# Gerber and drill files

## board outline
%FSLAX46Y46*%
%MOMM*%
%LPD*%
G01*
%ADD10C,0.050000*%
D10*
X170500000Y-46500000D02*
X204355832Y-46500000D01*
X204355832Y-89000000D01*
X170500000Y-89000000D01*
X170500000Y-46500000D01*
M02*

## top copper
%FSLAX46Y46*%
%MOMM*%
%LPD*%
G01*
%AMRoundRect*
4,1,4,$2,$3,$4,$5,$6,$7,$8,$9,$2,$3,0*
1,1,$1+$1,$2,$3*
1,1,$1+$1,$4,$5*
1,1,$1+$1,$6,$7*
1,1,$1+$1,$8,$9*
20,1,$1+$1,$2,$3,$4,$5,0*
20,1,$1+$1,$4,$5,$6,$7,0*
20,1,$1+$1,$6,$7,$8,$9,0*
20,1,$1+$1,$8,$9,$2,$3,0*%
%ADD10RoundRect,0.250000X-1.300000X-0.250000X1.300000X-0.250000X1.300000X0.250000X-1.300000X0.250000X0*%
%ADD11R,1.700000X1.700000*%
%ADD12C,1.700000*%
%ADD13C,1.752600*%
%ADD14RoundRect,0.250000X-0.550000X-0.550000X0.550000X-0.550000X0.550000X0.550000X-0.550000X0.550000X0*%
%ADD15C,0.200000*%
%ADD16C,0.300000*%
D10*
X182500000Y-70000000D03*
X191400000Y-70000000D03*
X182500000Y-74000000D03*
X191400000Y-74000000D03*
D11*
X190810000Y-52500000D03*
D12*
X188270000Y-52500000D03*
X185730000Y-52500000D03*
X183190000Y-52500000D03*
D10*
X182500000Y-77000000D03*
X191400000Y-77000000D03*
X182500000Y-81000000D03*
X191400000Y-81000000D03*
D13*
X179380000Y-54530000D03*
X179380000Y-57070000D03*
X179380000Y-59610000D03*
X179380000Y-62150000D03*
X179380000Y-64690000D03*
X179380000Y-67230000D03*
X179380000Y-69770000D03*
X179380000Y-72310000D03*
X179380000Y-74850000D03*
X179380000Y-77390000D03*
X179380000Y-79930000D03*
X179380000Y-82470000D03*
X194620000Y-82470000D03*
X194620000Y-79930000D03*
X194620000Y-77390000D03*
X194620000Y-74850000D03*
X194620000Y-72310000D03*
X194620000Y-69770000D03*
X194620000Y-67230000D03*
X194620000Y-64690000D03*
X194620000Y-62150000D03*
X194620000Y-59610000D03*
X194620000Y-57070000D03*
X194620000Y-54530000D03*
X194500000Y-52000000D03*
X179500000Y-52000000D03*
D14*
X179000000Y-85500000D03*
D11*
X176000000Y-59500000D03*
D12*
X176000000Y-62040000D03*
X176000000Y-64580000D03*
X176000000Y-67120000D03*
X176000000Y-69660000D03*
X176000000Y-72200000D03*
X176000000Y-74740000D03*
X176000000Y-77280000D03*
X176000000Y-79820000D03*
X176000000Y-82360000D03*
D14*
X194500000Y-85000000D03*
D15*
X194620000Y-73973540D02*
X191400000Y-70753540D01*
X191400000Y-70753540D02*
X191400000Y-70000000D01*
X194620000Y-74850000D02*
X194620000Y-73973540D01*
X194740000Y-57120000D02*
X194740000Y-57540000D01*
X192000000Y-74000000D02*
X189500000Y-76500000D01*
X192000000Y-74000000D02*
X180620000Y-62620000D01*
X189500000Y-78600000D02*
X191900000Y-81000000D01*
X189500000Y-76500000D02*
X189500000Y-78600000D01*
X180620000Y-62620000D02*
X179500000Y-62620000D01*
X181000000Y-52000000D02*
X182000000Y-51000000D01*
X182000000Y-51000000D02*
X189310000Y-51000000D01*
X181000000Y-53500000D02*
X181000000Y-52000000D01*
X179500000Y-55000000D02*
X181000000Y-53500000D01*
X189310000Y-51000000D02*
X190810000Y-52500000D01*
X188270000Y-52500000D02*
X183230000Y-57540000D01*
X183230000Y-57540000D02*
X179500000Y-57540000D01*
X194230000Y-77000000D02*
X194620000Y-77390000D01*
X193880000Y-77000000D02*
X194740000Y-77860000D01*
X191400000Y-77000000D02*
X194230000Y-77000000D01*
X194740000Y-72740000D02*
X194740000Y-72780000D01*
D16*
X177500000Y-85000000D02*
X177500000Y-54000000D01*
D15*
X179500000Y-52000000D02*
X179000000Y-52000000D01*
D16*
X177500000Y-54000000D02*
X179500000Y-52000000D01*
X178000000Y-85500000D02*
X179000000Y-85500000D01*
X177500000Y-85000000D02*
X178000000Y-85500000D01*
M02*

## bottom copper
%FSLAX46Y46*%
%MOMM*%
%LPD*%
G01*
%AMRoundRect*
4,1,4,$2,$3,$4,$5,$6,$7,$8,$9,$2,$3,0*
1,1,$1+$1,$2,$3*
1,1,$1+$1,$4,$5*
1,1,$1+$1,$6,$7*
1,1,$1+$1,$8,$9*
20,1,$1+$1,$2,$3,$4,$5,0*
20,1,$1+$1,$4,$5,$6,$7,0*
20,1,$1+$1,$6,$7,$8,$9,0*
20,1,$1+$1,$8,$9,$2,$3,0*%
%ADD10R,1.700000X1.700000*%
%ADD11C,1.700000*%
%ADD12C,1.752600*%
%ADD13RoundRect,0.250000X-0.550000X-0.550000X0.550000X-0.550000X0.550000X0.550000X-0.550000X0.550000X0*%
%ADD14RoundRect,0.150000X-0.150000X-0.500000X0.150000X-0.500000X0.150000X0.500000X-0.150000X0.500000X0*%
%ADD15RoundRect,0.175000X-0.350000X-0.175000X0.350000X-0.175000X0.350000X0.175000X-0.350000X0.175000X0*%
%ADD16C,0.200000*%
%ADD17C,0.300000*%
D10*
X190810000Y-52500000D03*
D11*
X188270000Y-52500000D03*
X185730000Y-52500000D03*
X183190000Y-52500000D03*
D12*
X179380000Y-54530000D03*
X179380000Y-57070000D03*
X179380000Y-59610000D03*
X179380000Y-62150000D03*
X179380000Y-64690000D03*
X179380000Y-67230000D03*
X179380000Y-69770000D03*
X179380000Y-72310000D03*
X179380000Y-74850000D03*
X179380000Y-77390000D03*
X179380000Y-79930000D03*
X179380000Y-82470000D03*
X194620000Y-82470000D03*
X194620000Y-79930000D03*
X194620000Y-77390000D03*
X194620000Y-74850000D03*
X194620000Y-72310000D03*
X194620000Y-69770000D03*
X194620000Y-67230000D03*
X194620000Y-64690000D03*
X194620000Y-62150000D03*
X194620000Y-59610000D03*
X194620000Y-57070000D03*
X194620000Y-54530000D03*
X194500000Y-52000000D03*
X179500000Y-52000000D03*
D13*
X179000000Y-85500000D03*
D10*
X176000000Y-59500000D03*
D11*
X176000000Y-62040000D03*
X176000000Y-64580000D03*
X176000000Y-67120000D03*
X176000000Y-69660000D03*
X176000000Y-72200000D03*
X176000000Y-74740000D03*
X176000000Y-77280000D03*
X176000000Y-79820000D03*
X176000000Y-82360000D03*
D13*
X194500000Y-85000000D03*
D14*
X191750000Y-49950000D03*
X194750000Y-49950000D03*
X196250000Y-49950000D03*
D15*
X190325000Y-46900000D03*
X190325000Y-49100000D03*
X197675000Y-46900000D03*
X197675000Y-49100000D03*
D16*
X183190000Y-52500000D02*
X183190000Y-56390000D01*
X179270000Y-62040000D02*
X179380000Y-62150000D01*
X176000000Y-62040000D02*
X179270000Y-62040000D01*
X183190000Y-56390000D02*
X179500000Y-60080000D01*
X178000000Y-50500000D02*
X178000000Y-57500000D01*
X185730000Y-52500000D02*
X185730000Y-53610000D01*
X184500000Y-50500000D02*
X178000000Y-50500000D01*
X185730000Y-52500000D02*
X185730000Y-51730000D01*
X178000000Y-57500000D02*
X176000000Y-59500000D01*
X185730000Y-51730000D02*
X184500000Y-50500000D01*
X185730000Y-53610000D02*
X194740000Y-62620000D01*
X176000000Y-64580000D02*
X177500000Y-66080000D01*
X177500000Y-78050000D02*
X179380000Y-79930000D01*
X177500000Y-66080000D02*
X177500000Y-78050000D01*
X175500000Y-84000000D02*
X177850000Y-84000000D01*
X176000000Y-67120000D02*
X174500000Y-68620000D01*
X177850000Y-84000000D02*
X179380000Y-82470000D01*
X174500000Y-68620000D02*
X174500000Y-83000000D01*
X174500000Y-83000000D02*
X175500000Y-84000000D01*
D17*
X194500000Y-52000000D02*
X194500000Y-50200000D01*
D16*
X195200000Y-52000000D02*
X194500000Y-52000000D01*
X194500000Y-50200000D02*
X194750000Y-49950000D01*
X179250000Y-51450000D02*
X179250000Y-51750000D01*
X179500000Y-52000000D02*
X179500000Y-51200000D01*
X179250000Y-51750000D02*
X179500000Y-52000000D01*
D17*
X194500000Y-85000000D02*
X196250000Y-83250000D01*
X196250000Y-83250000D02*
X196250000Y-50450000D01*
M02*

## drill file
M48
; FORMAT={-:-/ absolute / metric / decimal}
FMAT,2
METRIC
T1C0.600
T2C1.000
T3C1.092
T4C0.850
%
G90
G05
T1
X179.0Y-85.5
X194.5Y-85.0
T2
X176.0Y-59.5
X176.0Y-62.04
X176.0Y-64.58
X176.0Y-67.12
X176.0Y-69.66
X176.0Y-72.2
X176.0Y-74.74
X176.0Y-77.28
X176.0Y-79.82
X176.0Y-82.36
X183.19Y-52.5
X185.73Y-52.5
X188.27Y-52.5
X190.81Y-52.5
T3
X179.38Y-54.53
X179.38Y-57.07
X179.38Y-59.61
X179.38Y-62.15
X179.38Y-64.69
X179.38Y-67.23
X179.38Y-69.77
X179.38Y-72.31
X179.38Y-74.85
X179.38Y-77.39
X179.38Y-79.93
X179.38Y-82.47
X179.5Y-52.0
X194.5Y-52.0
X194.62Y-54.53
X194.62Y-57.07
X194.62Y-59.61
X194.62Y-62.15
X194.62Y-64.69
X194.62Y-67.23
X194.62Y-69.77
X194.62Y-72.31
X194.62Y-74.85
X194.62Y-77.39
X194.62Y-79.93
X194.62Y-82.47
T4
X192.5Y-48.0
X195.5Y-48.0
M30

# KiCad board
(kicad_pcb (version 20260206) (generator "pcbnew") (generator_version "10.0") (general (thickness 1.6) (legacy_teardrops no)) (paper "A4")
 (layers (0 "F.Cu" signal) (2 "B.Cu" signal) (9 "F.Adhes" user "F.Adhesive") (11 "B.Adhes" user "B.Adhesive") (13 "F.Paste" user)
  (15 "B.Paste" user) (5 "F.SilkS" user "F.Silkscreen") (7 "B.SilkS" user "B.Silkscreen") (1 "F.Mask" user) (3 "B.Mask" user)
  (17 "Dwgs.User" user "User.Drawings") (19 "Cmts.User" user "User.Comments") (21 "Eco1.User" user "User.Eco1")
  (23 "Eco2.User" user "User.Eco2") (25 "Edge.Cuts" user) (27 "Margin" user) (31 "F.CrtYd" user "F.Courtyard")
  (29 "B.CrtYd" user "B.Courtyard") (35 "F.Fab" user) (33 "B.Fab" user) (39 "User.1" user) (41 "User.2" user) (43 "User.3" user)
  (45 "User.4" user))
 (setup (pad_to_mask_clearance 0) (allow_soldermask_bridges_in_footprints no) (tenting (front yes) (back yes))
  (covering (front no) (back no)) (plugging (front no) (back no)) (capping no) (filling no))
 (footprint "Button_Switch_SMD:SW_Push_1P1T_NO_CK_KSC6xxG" (layer "F.Cu") (at 186.95 72)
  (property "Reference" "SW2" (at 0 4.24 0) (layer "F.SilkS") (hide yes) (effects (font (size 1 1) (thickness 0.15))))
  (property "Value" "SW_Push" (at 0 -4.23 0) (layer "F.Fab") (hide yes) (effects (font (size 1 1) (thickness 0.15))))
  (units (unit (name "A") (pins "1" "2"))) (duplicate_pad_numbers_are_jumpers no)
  (pad "1" smd roundrect (at -4.45 -2) (size 3.1 1) (layers "F.Cu" "F.Mask" "F.Paste") (roundrect_rratio 0.25) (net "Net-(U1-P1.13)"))
  (pad "1" smd roundrect (at 4.45 -2) (size 3.1 1) (layers "F.Cu" "F.Mask" "F.Paste") (roundrect_rratio 0.25) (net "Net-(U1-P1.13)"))
  (pad "2" smd roundrect (at -4.45 2) (size 3.1 1) (layers "F.Cu" "F.Mask" "F.Paste") (roundrect_rratio 0.25) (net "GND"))
  (pad "2" smd roundrect (at 4.45 2) (size 3.1 1) (layers "F.Cu" "F.Mask" "F.Paste") (roundrect_rratio 0.25) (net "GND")))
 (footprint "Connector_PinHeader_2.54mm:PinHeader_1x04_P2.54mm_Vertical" (layer "F.Cu") (at 190.81 52.5 -90)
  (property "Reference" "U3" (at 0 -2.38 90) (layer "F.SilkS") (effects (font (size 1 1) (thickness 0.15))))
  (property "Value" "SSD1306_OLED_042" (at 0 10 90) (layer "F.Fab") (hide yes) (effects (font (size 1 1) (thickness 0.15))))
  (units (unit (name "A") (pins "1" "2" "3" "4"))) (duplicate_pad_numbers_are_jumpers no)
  (pad "1" thru_hole rect (at 0 0 270) (size 1.7 1.7) (drill 1) (layers "*.Cu" "*.Mask") (remove_unused_layers no)
   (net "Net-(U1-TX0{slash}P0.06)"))
  (pad "2" thru_hole circle (at 0 2.54 270) (size 1.7 1.7) (drill 1) (layers "*.Cu" "*.Mask") (remove_unused_layers no)
   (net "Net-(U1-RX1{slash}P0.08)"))
  (pad "3" thru_hole circle (at 0 5.08 270) (size 1.7 1.7) (drill 1) (layers "*.Cu" "*.Mask") (remove_unused_layers no) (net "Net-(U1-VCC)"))
  (pad "4" thru_hole circle (at 0 7.62 270) (size 1.7 1.7) (drill 1) (layers "*.Cu" "*.Mask") (remove_unused_layers no) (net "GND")))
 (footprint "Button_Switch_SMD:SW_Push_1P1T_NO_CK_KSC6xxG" (layer "F.Cu") (at 186.95 79)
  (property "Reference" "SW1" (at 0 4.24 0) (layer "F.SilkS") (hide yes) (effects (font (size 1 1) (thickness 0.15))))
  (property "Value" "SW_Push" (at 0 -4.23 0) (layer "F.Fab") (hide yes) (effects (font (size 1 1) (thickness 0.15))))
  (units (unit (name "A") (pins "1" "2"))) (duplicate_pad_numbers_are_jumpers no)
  (pad "1" smd roundrect (at -4.45 -2) (size 3.1 1) (layers "F.Cu" "F.Mask" "F.Paste") (roundrect_rratio 0.25) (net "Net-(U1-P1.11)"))
  (pad "1" smd roundrect (at 4.45 -2) (size 3.1 1) (layers "F.Cu" "F.Mask" "F.Paste") (roundrect_rratio 0.25) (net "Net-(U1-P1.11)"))
  (pad "2" smd roundrect (at -4.45 2) (size 3.1 1) (layers "F.Cu" "F.Mask" "F.Paste") (roundrect_rratio 0.25) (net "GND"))
  (pad "2" smd roundrect (at 4.45 2) (size 3.1 1) (layers "F.Cu" "F.Mask" "F.Paste") (roundrect_rratio 0.25) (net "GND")))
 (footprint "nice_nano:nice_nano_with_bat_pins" (layer "F.Cu") (at 187 68.5 -90)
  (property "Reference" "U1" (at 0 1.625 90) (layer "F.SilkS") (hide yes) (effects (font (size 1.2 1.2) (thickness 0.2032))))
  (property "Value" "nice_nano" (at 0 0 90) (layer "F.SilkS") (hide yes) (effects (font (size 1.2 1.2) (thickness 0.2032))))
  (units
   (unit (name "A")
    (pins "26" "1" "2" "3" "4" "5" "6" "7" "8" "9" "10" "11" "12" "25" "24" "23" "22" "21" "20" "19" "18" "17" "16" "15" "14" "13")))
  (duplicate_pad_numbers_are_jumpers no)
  (pad "1" thru_hole circle (at -13.97 7.62 270) (size 1.7526 1.7526) (drill 1.0922) (layers "*.Cu" "*.SilkS" "*.Mask")
   (remove_unused_layers no) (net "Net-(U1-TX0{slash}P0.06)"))
  (pad "2" thru_hole circle (at -11.43 7.62 270) (size 1.7526 1.7526) (drill 1.0922) (layers "*.Cu" "*.SilkS" "*.Mask")
   (remove_unused_layers no) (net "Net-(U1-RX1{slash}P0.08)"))
  (pad "3" thru_hole circle (at -8.89 7.62 270) (size 1.7526 1.7526) (drill 1.0922) (layers "*.Cu" "*.SilkS" "*.Mask")
   (remove_unused_layers no) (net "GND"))
  (pad "4" thru_hole circle (at -6.35 7.62 270) (size 1.7526 1.7526) (drill 1.0922) (layers "*.Cu" "*.SilkS" "*.Mask")
   (remove_unused_layers no) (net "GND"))
  (pad "5" thru_hole circle (at -3.81 7.62 270) (size 1.7526 1.7526) (drill 1.0922) (layers "*.Cu" "*.SilkS" "*.Mask")
   (remove_unused_layers no) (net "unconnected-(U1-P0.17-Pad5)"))
  (pad "6" thru_hole circle (at -1.27 7.62 270) (size 1.7526 1.7526) (drill 1.0922) (layers "*.Cu" "*.SilkS" "*.Mask")
   (remove_unused_layers no) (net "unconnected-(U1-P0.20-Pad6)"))
  (pad "7" thru_hole circle (at 1.27 7.62 270) (size 1.7526 1.7526) (drill 1.0922) (layers "*.Cu" "*.SilkS" "*.Mask")
   (remove_unused_layers no) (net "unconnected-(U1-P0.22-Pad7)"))
  (pad "8" thru_hole circle (at 3.81 7.62 270) (size 1.7526 1.7526) (drill 1.0922) (layers "*.Cu" "*.SilkS" "*.Mask")
   (remove_unused_layers no) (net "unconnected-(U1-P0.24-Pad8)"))
  (pad "9" thru_hole circle (at 6.35 7.62 270) (size 1.7526 1.7526) (drill 1.0922) (layers "*.Cu" "*.SilkS" "*.Mask")
   (remove_unused_layers no) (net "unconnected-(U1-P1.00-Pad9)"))
  (pad "10" thru_hole circle (at 8.89 7.62 270) (size 1.7526 1.7526) (drill 1.0922) (layers "*.Cu" "*.SilkS" "*.Mask")
   (remove_unused_layers no) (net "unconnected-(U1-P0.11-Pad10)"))
  (pad "11" thru_hole circle (at 11.43 7.62 270) (size 1.7526 1.7526) (drill 1.0922) (layers "*.Cu" "*.SilkS" "*.Mask")
   (remove_unused_layers no) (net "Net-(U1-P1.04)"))
  (pad "12" thru_hole circle (at 13.97 7.62 270) (size 1.7526 1.7526) (drill 1.0922) (layers "*.Cu" "*.SilkS" "*.Mask")
   (remove_unused_layers no) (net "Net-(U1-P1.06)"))
  (pad "13" thru_hole circle (at 13.97 -7.62 270) (size 1.7526 1.7526) (drill 1.0922) (layers "*.Cu" "*.SilkS" "*.Mask")
   (remove_unused_layers no) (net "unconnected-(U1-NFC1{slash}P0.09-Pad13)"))
  (pad "14" thru_hole circle (at 11.43 -7.62 270) (size 1.7526 1.7526) (drill 1.0922) (layers "*.Cu" "*.SilkS" "*.Mask")
   (remove_unused_layers no) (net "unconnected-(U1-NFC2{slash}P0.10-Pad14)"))
  (pad "15" thru_hole circle (at 8.89 -7.62 270) (size 1.7526 1.7526) (drill 1.0922) (layers "*.Cu" "*.SilkS" "*.Mask")
   (remove_unused_layers no) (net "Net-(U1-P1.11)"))
  (pad "16" thru_hole circle (at 6.35 -7.62 270) (size 1.7526 1.7526) (drill 1.0922) (layers "*.Cu" "*.SilkS" "*.Mask")
   (remove_unused_layers no) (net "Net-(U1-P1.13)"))
  (pad "17" thru_hole circle (at 3.81 -7.62 270) (size 1.7526 1.7526) (drill 1.0922) (layers "*.Cu" "*.SilkS" "*.Mask")
   (remove_unused_layers no) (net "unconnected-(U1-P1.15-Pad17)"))
  (pad "18" thru_hole circle (at 1.27 -7.62 270) (size 1.7526 1.7526) (drill 1.0922) (layers "*.Cu" "*.SilkS" "*.Mask")
   (remove_unused_layers no) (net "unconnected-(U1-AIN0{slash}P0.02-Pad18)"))
  (pad "19" thru_hole circle (at -1.27 -7.62 270) (size 1.7526 1.7526) (drill 1.0922) (layers "*.Cu" "*.SilkS" "*.Mask")
   (remove_unused_layers no) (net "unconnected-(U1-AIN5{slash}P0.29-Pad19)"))
  (pad "20" thru_hole circle (at -3.81 -7.62 270) (size 1.7526 1.7526) (drill 1.0922) (layers "*.Cu" "*.SilkS" "*.Mask")
   (remove_unused_layers no) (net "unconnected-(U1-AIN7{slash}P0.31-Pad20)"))
  (pad "21" thru_hole circle (at -6.35 -7.62 270) (size 1.7526 1.7526) (drill 1.0922) (layers "*.Cu" "*.SilkS" "*.Mask")
   (remove_unused_layers no) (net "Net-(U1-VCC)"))
  (pad "22" thru_hole circle (at -8.89 -7.62 270) (size 1.7526 1.7526) (drill 1.0922) (layers "*.Cu" "*.SilkS" "*.Mask")
   (remove_unused_layers no) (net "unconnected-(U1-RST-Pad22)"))
  (pad "23" thru_hole circle (at -11.43 -7.62 270) (size 1.7526 1.7526) (drill 1.0922) (layers "*.Cu" "*.SilkS" "*.Mask")
   (remove_unused_layers no) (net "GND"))
  (pad "24" thru_hole circle (at -13.97 -7.62 270) (size 1.7526 1.7526) (drill 1.0922) (layers "*.Cu" "*.SilkS" "*.Mask")
   (remove_unused_layers no) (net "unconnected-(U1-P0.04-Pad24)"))
  (pad "25" thru_hole circle (at -16.5 -7.5 270) (size 1.7526 1.7526) (drill 1.0922) (layers "*.Cu" "*.SilkS" "*.Mask")
   (remove_unused_layers no) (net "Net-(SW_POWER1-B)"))
  (pad "26" thru_hole circle (at -16.5 7.5 270) (size 1.7526 1.7526) (drill 1.0922) (layers "*.Cu" "*.SilkS" "*.Mask")
   (remove_unused_layers no) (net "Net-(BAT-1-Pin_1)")))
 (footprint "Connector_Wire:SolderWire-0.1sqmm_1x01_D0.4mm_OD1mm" (layer "B.Cu") (at 179 85.5)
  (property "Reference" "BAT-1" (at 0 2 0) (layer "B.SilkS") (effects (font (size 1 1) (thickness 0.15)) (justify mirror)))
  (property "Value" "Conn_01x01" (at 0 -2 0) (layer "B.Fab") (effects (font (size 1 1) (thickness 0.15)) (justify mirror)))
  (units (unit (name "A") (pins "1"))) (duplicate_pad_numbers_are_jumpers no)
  (pad "1" thru_hole roundrect (at 0 0) (size 1.6 1.6) (drill 0.6) (layers "*.Cu" "*.Mask") (remove_unused_layers no)
   (roundrect_rratio 0.15625) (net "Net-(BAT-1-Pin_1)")))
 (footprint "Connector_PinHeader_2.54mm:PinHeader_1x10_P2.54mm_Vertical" (layer "B.Cu") (at 176 59.5 180)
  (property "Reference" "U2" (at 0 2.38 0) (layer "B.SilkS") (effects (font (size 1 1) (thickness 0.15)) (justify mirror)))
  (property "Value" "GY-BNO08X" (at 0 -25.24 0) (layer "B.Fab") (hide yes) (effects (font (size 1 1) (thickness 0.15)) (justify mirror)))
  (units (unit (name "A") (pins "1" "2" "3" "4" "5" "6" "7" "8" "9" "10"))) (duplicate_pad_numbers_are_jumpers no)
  (pad "1" thru_hole rect (at 0 0 180) (size 1.7 1.7) (drill 1) (layers "*.Cu" "*.Mask") (remove_unused_layers no) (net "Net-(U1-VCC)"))
  (pad "2" thru_hole circle (at 0 -2.54 180) (size 1.7 1.7) (drill 1) (layers "*.Cu" "*.Mask") (remove_unused_layers no) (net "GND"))
  (pad "3" thru_hole circle (at 0 -5.08 180) (size 1.7 1.7) (drill 1) (layers "*.Cu" "*.Mask") (remove_unused_layers no)
   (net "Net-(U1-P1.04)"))
  (pad "4" thru_hole circle (at 0 -7.62 180) (size 1.7 1.7) (drill 1) (layers "*.Cu" "*.Mask") (remove_unused_layers no)
   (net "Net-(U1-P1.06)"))
  (pad "5" thru_hole circle (at 0 -10.16 180) (size 1.7 1.7) (drill 1) (layers "*.Cu" "*.Mask") (remove_unused_layers no)
   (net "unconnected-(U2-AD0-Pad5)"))
  (pad "6" thru_hole circle (at 0 -12.7 180) (size 1.7 1.7) (drill 1) (layers "*.Cu" "*.Mask") (remove_unused_layers no)
   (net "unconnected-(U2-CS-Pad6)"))
  (pad "7" thru_hole circle (at 0 -15.24 180) (size 1.7 1.7) (drill 1) (layers "*.Cu" "*.Mask") (remove_unused_layers no)
   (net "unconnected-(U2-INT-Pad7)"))
  (pad "8" thru_hole circle (at 0 -17.78 180) (size 1.7 1.7) (drill 1) (layers "*.Cu" "*.Mask") (remove_unused_layers no)
   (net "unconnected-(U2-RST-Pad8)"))
  (pad "9" thru_hole circle (at 0 -20.32 180) (size 1.7 1.7) (drill 1) (layers "*.Cu" "*.Mask") (remove_unused_layers no)
   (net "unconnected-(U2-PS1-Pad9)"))
  (pad "10" thru_hole circle (at 0 -22.86 180) (size 1.7 1.7) (drill 1) (layers "*.Cu" "*.Mask") (remove_unused_layers no)
   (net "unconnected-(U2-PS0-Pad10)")))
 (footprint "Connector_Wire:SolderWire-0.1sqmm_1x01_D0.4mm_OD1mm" (layer "B.Cu") (at 194.5 85)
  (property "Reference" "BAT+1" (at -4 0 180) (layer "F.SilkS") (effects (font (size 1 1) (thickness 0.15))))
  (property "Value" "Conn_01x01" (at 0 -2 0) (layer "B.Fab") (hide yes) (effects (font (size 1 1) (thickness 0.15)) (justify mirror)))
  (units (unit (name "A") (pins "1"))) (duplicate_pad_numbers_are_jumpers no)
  (pad "1" thru_hole roundrect (at 0 0) (size 1.6 1.6) (drill 0.6) (layers "*.Cu" "*.Mask") (remove_unused_layers no)
   (roundrect_rratio 0.15625) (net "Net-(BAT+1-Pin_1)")))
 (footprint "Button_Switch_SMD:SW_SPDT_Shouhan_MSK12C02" (layer "B.Cu") (at 194 48)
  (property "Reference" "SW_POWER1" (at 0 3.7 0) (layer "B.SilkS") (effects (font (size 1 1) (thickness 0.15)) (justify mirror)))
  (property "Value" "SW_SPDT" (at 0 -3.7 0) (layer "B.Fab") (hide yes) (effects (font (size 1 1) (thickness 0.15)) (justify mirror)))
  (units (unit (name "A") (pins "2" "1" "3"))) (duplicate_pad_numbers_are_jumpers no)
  (pad "" np_thru_hole circle (at -1.5 0) (size 0.85 0.85) (drill 0.85) (layers "*.Mask"))
  (pad "" np_thru_hole circle (at 1.5 0) (size 0.85 0.85) (drill 0.85) (layers "*.Mask"))
  (pad "1" smd roundrect (at -2.25 1.95) (size 0.6 1.3) (layers "B.Cu" "B.Mask" "B.Paste") (roundrect_rratio 0.25)
   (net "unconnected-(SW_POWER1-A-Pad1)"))
  (pad "2" smd roundrect (at 0.75 1.95) (size 0.6 1.3) (layers "B.Cu" "B.Mask" "B.Paste") (roundrect_rratio 0.25) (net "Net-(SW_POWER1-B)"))
  (pad "3" smd roundrect (at 2.25 1.95) (size 0.6 1.3) (layers "B.Cu" "B.Mask" "B.Paste") (roundrect_rratio 0.25) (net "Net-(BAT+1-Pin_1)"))
  (pad "SH" smd roundrect (at -3.675 -1.1) (size 1.05 0.7) (layers "B.Cu" "B.Mask" "B.Paste") (roundrect_rratio 0.25))
  (pad "SH" smd roundrect (at -3.675 1.1) (size 1.05 0.7) (layers "B.Cu" "B.Mask" "B.Paste") (roundrect_rratio 0.25))
  (pad "SH" smd roundrect (at 3.675 -1.1) (size 1.05 0.7) (layers "B.Cu" "B.Mask" "B.Paste") (roundrect_rratio 0.25))
  (pad "SH" smd roundrect (at 3.675 1.1) (size 1.05 0.7) (layers "B.Cu" "B.Mask" "B.Paste") (roundrect_rratio 0.25)))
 (gr_rect (start 170.5 46.5) (end 204.355832 89) (stroke (width 0.05) (type default)) (fill no) (layer "Edge.Cuts"))
 (segment (start 194.62 73.97354) (end 191.4 70.75354) (width 0.2) (layer "F.Cu") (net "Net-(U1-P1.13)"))
 (segment (start 191.4 70.75354) (end 191.4 70) (width 0.2) (layer "F.Cu") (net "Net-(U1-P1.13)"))
 (segment (start 194.62 74.85) (end 194.62 73.97354) (width 0.2) (layer "F.Cu") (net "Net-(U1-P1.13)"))
 (segment (start 194.74 57.12) (end 194.74 57.54) (width 0.2) (layer "F.Cu") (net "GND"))
 (segment (start 192 74) (end 189.5 76.5) (width 0.2) (layer "F.Cu") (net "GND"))
 (segment (start 192 74) (end 180.62 62.62) (width 0.2) (layer "F.Cu") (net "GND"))
 (segment (start 189.5 78.6) (end 191.9 81) (width 0.2) (layer "F.Cu") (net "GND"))
 (segment (start 189.5 76.5) (end 189.5 78.6) (width 0.2) (layer "F.Cu") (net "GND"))
 (segment (start 180.62 62.62) (end 179.5 62.62) (width 0.2) (layer "F.Cu") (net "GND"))
 (segment (start 183.19 52.5) (end 183.19 56.39) (width 0.2) (layer "B.Cu") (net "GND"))
 (segment (start 179.27 62.04) (end 179.38 62.15) (width 0.2) (layer "B.Cu") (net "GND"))
 (segment (start 176 62.04) (end 179.27 62.04) (width 0.2) (layer "B.Cu") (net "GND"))
 (segment (start 183.19 56.39) (end 179.5 60.08) (width 0.2) (layer "B.Cu") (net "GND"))
 (segment (start 181 52) (end 182 51) (width 0.2) (layer "F.Cu") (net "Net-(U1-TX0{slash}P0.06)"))
 (segment (start 182 51) (end 189.31 51) (width 0.2) (layer "F.Cu") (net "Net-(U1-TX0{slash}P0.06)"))
 (segment (start 181 53.5) (end 181 52) (width 0.2) (layer "F.Cu") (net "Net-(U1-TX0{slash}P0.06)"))
 (segment (start 179.5 55) (end 181 53.5) (width 0.2) (layer "F.Cu") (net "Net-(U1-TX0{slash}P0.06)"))
 (segment (start 189.31 51) (end 190.81 52.5) (width 0.2) (layer "F.Cu") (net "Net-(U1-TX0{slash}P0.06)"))
 (segment (start 188.27 52.5) (end 183.23 57.54) (width 0.2) (layer "F.Cu") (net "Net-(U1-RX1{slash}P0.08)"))
 (segment (start 183.23 57.54) (end 179.5 57.54) (width 0.2) (layer "F.Cu") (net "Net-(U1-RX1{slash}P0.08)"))
 (segment (start 178 50.5) (end 178 57.5) (width 0.2) (layer "B.Cu") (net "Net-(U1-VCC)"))
 (segment (start 185.73 52.5) (end 185.73 53.61) (width 0.2) (layer "B.Cu") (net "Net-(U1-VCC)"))
 (segment (start 184.5 50.5) (end 178 50.5) (width 0.2) (layer "B.Cu") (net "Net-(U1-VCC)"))
 (segment (start 185.73 52.5) (end 185.73 51.73) (width 0.2) (layer "B.Cu") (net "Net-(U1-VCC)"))
 (segment (start 178 57.5) (end 176 59.5) (width 0.2) (layer "B.Cu") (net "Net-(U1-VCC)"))
 (segment (start 185.73 51.73) (end 184.5 50.5) (width 0.2) (layer "B.Cu") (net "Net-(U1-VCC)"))
 (segment (start 185.73 53.61) (end 194.74 62.62) (width 0.2) (layer "B.Cu") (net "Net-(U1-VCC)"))
 (segment (start 194.23 77) (end 194.62 77.39) (width 0.2) (layer "F.Cu") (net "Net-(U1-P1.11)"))
 (segment (start 193.88 77) (end 194.74 77.86) (width 0.2) (layer "F.Cu") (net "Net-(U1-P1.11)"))
 (segment (start 191.4 77) (end 194.23 77) (width 0.2) (layer "F.Cu") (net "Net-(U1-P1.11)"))
 (segment (start 176 64.58) (end 177.5 66.08) (width 0.2) (layer "B.Cu") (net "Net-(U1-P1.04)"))
 (segment (start 177.5 78.05) (end 179.38 79.93) (width 0.2) (layer "B.Cu") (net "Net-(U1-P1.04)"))
 (segment (start 177.5 66.08) (end 177.5 78.05) (width 0.2) (layer "B.Cu") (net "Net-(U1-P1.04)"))
 (segment (start 175.5 84) (end 177.85 84) (width 0.2) (layer "B.Cu") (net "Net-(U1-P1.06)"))
 (segment (start 176 67.12) (end 174.5 68.62) (width 0.2) (layer "B.Cu") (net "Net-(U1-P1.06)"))
 (segment (start 177.85 84) (end 179.38 82.47) (width 0.2) (layer "B.Cu") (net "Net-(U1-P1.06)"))
 (segment (start 174.5 68.62) (end 174.5 83) (width 0.2) (layer "B.Cu") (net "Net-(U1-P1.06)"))
 (segment (start 174.5 83) (end 175.5 84) (width 0.2) (layer "B.Cu") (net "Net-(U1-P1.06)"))
 (segment (start 194.74 72.74) (end 194.74 72.78) (width 0.2) (layer "F.Cu") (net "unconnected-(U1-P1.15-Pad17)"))
 (segment (start 194.5 52) (end 194.5 50.2) (width 0.3) (layer "B.Cu") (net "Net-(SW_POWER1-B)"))
 (segment (start 195.2 52) (end 194.5 52) (width 0.2) (layer "B.Cu") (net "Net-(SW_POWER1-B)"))
 (segment (start 194.5 50.2) (end 194.75 49.95) (width 0.2) (layer "B.Cu") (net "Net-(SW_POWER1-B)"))
 (segment (start 177.5 85) (end 177.5 54) (width 0.3) (layer "F.Cu") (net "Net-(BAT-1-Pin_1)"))
 (segment (start 179.5 52) (end 179 52) (width 0.2) (layer "F.Cu") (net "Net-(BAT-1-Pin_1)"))
 (segment (start 177.5 54) (end 179.5 52) (width 0.3) (layer "F.Cu") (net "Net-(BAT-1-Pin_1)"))
 (segment (start 178 85.5) (end 179 85.5) (width 0.3) (layer "F.Cu") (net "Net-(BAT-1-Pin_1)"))
 (segment (start 177.5 85) (end 178 85.5) (width 0.3) (layer "F.Cu") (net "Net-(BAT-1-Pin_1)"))
 (segment (start 179.25 51.45) (end 179.25 51.75) (width 0.2) (layer "B.Cu") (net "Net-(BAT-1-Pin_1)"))
 (segment (start 179.5 52) (end 179.5 51.2) (width 0.2) (layer "B.Cu") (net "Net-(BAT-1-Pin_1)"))
 (segment (start 179.25 51.75) (end 179.5 52) (width 0.2) (layer "B.Cu") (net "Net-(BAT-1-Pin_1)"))
 (segment (start 194.5 85) (end 196.25 83.25) (width 0.3) (layer "B.Cu") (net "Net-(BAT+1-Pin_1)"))
 (segment (start 196.25 83.25) (end 196.25 50.45) (width 0.3) (layer "B.Cu") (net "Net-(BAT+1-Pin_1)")))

